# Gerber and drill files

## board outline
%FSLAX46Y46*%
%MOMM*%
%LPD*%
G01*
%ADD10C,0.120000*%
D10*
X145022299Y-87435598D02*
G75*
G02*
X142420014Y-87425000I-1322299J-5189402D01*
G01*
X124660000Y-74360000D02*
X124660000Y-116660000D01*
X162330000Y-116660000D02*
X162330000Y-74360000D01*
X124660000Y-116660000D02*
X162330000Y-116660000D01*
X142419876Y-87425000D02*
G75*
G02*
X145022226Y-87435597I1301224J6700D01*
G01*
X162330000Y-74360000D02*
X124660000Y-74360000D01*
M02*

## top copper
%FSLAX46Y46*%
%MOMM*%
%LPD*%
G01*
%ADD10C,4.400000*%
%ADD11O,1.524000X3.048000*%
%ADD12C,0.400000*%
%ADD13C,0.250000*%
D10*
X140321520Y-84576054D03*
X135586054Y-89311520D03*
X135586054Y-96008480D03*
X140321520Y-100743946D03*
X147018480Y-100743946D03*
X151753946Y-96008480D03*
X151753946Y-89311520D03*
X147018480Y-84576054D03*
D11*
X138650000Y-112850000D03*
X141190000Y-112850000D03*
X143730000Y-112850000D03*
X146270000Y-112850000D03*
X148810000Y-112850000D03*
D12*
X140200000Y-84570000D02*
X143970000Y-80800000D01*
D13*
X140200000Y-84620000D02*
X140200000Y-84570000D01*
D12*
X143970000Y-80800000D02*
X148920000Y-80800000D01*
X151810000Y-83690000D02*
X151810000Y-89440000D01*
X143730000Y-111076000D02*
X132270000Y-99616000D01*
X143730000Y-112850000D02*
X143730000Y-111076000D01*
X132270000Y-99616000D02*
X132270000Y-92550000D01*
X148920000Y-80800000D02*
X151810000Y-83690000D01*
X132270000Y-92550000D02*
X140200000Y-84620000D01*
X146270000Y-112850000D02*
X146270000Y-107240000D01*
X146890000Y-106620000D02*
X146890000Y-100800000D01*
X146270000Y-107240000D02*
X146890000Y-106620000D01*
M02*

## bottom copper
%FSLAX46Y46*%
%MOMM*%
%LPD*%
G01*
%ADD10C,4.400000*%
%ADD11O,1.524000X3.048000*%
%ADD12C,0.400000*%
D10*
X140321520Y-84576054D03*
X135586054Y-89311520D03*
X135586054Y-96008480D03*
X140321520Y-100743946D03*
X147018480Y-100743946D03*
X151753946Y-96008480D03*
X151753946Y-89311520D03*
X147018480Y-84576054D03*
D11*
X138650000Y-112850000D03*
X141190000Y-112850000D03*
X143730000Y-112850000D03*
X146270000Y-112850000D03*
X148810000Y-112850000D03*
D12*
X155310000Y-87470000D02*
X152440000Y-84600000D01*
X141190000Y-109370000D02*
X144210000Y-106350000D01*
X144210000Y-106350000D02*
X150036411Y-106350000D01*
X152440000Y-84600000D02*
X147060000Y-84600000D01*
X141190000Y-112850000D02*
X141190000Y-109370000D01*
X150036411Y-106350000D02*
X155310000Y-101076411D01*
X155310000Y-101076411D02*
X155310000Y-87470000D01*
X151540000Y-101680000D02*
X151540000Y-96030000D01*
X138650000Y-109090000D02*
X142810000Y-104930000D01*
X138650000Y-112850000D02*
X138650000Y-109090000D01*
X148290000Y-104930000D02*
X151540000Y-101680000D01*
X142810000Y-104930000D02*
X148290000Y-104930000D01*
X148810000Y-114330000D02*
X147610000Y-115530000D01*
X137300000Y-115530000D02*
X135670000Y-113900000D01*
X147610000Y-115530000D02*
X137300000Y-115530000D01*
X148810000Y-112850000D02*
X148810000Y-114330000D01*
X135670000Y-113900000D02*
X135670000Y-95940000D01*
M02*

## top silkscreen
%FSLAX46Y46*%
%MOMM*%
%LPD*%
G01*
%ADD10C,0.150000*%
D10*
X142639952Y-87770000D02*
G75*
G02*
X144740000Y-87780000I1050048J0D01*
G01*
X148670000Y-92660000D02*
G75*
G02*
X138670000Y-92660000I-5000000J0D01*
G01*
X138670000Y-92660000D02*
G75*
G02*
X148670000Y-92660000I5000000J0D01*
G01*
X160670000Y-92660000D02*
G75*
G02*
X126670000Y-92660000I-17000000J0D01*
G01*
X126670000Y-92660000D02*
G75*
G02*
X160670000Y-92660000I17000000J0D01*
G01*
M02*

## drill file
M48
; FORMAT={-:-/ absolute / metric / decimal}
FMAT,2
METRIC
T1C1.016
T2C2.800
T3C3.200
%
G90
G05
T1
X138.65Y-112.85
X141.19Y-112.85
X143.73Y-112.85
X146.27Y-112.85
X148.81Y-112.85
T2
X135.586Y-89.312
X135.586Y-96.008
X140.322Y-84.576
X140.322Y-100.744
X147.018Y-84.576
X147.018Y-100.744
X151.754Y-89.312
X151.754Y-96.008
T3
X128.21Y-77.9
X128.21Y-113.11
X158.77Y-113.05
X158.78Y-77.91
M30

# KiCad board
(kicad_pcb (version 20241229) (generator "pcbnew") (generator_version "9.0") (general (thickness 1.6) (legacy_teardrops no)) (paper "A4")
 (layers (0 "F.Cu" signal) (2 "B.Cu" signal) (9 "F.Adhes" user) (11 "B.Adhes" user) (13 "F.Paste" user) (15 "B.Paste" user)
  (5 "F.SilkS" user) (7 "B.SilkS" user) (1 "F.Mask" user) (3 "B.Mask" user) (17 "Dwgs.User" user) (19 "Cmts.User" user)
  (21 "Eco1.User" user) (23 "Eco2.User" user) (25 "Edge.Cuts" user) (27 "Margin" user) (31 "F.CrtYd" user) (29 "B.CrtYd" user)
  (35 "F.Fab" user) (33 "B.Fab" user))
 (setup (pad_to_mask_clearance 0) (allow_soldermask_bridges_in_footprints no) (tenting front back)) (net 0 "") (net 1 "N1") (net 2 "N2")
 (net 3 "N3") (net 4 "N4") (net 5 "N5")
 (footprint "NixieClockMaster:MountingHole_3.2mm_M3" (layer "F.Cu") (at 128.21 77.9)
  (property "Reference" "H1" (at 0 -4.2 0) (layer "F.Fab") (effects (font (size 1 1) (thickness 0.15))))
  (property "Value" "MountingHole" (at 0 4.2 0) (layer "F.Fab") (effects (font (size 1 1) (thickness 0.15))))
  (pad "" np_thru_hole circle (at 0 0) (size 3.2 3.2) (drill 3.2) (layers "*.Cu" "*.Mask")))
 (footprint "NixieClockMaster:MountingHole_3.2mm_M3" (layer "F.Cu") (at 128.21 113.11)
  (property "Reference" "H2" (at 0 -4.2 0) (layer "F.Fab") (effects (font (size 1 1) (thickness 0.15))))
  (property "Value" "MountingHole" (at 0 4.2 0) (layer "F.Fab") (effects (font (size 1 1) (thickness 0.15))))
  (pad "" np_thru_hole circle (at 0 0) (size 3.2 3.2) (drill 3.2) (layers "*.Cu" "*.Mask")))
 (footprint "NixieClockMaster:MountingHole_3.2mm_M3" (layer "F.Cu") (at 158.78 77.91)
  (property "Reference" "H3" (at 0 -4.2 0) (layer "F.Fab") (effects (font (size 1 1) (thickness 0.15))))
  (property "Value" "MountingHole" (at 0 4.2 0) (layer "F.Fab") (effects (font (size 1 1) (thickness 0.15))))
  (pad "" np_thru_hole circle (at 0 0) (size 3.2 3.2) (drill 3.2) (layers "*.Cu" "*.Mask")))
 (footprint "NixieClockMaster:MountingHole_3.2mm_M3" (layer "F.Cu") (at 158.77 113.05)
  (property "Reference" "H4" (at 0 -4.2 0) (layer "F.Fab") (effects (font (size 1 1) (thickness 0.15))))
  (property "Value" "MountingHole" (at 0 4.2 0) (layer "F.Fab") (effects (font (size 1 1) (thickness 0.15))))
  (pad "" np_thru_hole circle (at 0 0) (size 3.2 3.2) (drill 3.2) (layers "*.Cu" "*.Mask")))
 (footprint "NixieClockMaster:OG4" (layer "F.Cu") (at 143.67 92.66)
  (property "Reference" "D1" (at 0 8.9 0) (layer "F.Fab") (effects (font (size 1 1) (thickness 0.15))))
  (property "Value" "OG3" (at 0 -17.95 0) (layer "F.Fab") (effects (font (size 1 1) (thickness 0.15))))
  (fp_arc (start -1.030048 -4.89) (mid 0.025 -5.940036) (end 1.07 -4.88) (stroke (width 0.15) (type solid)) (layer "F.SilkS"))
  (fp_circle (center 0 0) (end 5 0) (stroke (width 0.15) (type solid)) (fill no) (layer "F.SilkS"))
  (fp_circle (center 0 0) (end 17 0) (stroke (width 0.15) (type solid)) (fill no) (layer "F.SilkS"))
  (pad "1" thru_hole circle (at -3.34848 -8.083946) (size 4.4 4.4) (drill 2.8) (layers "*.Cu" "*.Mask") (remove_unused_layers no)
   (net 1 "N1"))
  (pad "2" thru_hole circle (at -8.083946 -3.34848) (size 4.4 4.4) (drill 2.8) (layers "*.Cu" "*.Mask") (remove_unused_layers no)
   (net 1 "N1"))
  (pad "3" thru_hole circle (at -8.083946 3.34848) (size 4.4 4.4) (drill 2.8) (layers "*.Cu" "*.Mask") (remove_unused_layers no)
   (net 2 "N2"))
  (pad "4" thru_hole circle (at -3.34848 8.083946) (size 4.4 4.4) (drill 2.8) (layers "*.Cu" "*.Mask") (remove_unused_layers no))
  (pad "5" thru_hole circle (at 3.34848 8.083946) (size 4.4 4.4) (drill 2.8) (layers "*.Cu" "*.Mask") (remove_unused_layers no) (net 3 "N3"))
  (pad "6" thru_hole circle (at 8.083946 3.34848) (size 4.4 4.4) (drill 2.8) (layers "*.Cu" "*.Mask") (remove_unused_layers no) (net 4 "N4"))
  (pad "7" thru_hole circle (at 8.083946 -3.34848) (size 4.4 4.4) (drill 2.8) (layers "*.Cu" "*.Mask") (remove_unused_layers no)
   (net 1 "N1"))
  (pad "8" thru_hole circle (at 3.34848 -8.083946) (size 4.4 4.4) (drill 2.8) (layers "*.Cu" "*.Mask") (remove_unused_layers no)
   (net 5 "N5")))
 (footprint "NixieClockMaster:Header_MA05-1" (layer "B.Cu") (at 145 112.85)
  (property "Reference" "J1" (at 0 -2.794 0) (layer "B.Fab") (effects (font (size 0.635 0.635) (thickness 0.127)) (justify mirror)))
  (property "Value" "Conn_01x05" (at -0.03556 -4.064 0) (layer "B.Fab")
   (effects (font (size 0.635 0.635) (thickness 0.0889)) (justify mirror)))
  (pad "1" thru_hole oval (at -6.35 0 180) (size 1.524 3.048) (drill 1.016) (layers "*.Cu" "*.Mask" "B.SilkS") (remove_unused_layers no)
   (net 4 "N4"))
  (pad "2" thru_hole oval (at -3.81 0 180) (size 1.524 3.048) (drill 1.016) (layers "*.Cu" "*.Mask" "B.SilkS") (remove_unused_layers no)
   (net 5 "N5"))
  (pad "3" thru_hole oval (at -1.27 0 180) (size 1.524 3.048) (drill 1.016) (layers "*.Cu" "*.Mask" "B.SilkS") (remove_unused_layers no)
   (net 1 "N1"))
  (pad "4" thru_hole oval (at 1.27 0 180) (size 1.524 3.048) (drill 1.016) (layers "*.Cu" "*.Mask" "B.SilkS") (remove_unused_layers no)
   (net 3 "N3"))
  (pad "5" thru_hole oval (at 3.81 0 180) (size 1.524 3.048) (drill 1.016) (layers "*.Cu" "*.Mask" "B.SilkS") (remove_unused_layers no)
   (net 2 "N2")))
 (gr_arc (start 145.022299 87.435598) (mid 143.67819 97.980174) (end 142.420014 87.425) (stroke (width 0.12) (type solid))
  (layer "Edge.Cuts"))
 (gr_line (start 124.66 74.36) (end 124.66 116.66) (stroke (width 0.12) (type solid)) (layer "Edge.Cuts"))
 (gr_line (start 162.33 116.66) (end 162.33 74.36) (stroke (width 0.12) (type solid)) (layer "Edge.Cuts"))
 (gr_line (start 124.66 116.66) (end 162.33 116.66) (stroke (width 0.12) (type solid)) (layer "Edge.Cuts"))
 (gr_arc (start 142.419876 87.425) (mid 143.726435 86.117072) (end 145.022299 87.435598) (stroke (width 0.12) (type solid))
  (layer "Edge.Cuts"))
 (gr_line (start 162.33 74.36) (end 124.66 74.36) (stroke (width 0.12) (type solid)) (layer "Edge.Cuts"))
 (segment (start 155.31 87.47) (end 152.44 84.6) (width 0.4) (layer "B.Cu") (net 5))
 (segment (start 141.19 109.37) (end 144.21 106.35) (width 0.4) (layer "B.Cu") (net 5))
 (segment (start 144.21 106.35) (end 150.036411 106.35) (width 0.4) (layer "B.Cu") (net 5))
 (segment (start 152.44 84.6) (end 147.06 84.6) (width 0.4) (layer "B.Cu") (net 5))
 (segment (start 141.19 112.85) (end 141.19 109.37) (width 0.4) (layer "B.Cu") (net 5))
 (segment (start 150.036411 106.35) (end 155.31 101.076411) (width 0.4) (layer "B.Cu") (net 5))
 (segment (start 155.31 101.076411) (end 155.31 87.47) (width 0.4) (layer "B.Cu") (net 5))
 (segment (start 151.54 101.68) (end 151.54 96.03) (width 0.4) (layer "B.Cu") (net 4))
 (segment (start 138.65 109.09) (end 142.81 104.93) (width 0.4) (layer "B.Cu") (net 4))
 (segment (start 138.65 112.85) (end 138.65 109.09) (width 0.4) (layer "B.Cu") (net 4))
 (segment (start 148.29 104.93) (end 151.54 101.68) (width 0.4) (layer "B.Cu") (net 4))
 (segment (start 142.81 104.93) (end 148.29 104.93) (width 0.4) (layer "B.Cu") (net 4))
 (segment (start 148.81 114.33) (end 147.61 115.53) (width 0.4) (layer "B.Cu") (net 2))
 (segment (start 137.3 115.53) (end 135.67 113.9) (width 0.4) (layer "B.Cu") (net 2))
 (segment (start 147.61 115.53) (end 137.3 115.53) (width 0.4) (layer "B.Cu") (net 2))
 (segment (start 148.81 112.85) (end 148.81 114.33) (width 0.4) (layer "B.Cu") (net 2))
 (segment (start 135.67 113.9) (end 135.67 95.94) (width 0.4) (layer "B.Cu") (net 2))
 (segment (start 140.2 84.57) (end 143.97 80.8) (width 0.4) (layer "F.Cu") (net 1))
 (segment (start 140.2 84.62) (end 140.2 84.57) (width 0.25) (layer "F.Cu") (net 1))
 (segment (start 143.97 80.8) (end 148.92 80.8) (width 0.4) (layer "F.Cu") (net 1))
 (segment (start 151.81 83.69) (end 151.81 89.44) (width 0.4) (layer "F.Cu") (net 1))
 (segment (start 143.73 111.076) (end 132.27 99.616) (width 0.4) (layer "F.Cu") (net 1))
 (segment (start 143.73 112.85) (end 143.73 111.076) (width 0.4) (layer "F.Cu") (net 1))
 (segment (start 132.27 99.616) (end 132.27 92.55) (width 0.4) (layer "F.Cu") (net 1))
 (segment (start 148.92 80.8) (end 151.81 83.69) (width 0.4) (layer "F.Cu") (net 1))
 (segment (start 132.27 92.55) (end 140.2 84.62) (width 0.4) (layer "F.Cu") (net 1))
 (segment (start 146.27 112.85) (end 146.27 107.24) (width 0.4) (layer "F.Cu") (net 3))
 (segment (start 146.89 106.62) (end 146.89 100.8) (width 0.4) (layer "F.Cu") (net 3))
 (segment (start 146.27 107.24) (end 146.89 106.62) (width 0.4) (layer "F.Cu") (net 3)))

